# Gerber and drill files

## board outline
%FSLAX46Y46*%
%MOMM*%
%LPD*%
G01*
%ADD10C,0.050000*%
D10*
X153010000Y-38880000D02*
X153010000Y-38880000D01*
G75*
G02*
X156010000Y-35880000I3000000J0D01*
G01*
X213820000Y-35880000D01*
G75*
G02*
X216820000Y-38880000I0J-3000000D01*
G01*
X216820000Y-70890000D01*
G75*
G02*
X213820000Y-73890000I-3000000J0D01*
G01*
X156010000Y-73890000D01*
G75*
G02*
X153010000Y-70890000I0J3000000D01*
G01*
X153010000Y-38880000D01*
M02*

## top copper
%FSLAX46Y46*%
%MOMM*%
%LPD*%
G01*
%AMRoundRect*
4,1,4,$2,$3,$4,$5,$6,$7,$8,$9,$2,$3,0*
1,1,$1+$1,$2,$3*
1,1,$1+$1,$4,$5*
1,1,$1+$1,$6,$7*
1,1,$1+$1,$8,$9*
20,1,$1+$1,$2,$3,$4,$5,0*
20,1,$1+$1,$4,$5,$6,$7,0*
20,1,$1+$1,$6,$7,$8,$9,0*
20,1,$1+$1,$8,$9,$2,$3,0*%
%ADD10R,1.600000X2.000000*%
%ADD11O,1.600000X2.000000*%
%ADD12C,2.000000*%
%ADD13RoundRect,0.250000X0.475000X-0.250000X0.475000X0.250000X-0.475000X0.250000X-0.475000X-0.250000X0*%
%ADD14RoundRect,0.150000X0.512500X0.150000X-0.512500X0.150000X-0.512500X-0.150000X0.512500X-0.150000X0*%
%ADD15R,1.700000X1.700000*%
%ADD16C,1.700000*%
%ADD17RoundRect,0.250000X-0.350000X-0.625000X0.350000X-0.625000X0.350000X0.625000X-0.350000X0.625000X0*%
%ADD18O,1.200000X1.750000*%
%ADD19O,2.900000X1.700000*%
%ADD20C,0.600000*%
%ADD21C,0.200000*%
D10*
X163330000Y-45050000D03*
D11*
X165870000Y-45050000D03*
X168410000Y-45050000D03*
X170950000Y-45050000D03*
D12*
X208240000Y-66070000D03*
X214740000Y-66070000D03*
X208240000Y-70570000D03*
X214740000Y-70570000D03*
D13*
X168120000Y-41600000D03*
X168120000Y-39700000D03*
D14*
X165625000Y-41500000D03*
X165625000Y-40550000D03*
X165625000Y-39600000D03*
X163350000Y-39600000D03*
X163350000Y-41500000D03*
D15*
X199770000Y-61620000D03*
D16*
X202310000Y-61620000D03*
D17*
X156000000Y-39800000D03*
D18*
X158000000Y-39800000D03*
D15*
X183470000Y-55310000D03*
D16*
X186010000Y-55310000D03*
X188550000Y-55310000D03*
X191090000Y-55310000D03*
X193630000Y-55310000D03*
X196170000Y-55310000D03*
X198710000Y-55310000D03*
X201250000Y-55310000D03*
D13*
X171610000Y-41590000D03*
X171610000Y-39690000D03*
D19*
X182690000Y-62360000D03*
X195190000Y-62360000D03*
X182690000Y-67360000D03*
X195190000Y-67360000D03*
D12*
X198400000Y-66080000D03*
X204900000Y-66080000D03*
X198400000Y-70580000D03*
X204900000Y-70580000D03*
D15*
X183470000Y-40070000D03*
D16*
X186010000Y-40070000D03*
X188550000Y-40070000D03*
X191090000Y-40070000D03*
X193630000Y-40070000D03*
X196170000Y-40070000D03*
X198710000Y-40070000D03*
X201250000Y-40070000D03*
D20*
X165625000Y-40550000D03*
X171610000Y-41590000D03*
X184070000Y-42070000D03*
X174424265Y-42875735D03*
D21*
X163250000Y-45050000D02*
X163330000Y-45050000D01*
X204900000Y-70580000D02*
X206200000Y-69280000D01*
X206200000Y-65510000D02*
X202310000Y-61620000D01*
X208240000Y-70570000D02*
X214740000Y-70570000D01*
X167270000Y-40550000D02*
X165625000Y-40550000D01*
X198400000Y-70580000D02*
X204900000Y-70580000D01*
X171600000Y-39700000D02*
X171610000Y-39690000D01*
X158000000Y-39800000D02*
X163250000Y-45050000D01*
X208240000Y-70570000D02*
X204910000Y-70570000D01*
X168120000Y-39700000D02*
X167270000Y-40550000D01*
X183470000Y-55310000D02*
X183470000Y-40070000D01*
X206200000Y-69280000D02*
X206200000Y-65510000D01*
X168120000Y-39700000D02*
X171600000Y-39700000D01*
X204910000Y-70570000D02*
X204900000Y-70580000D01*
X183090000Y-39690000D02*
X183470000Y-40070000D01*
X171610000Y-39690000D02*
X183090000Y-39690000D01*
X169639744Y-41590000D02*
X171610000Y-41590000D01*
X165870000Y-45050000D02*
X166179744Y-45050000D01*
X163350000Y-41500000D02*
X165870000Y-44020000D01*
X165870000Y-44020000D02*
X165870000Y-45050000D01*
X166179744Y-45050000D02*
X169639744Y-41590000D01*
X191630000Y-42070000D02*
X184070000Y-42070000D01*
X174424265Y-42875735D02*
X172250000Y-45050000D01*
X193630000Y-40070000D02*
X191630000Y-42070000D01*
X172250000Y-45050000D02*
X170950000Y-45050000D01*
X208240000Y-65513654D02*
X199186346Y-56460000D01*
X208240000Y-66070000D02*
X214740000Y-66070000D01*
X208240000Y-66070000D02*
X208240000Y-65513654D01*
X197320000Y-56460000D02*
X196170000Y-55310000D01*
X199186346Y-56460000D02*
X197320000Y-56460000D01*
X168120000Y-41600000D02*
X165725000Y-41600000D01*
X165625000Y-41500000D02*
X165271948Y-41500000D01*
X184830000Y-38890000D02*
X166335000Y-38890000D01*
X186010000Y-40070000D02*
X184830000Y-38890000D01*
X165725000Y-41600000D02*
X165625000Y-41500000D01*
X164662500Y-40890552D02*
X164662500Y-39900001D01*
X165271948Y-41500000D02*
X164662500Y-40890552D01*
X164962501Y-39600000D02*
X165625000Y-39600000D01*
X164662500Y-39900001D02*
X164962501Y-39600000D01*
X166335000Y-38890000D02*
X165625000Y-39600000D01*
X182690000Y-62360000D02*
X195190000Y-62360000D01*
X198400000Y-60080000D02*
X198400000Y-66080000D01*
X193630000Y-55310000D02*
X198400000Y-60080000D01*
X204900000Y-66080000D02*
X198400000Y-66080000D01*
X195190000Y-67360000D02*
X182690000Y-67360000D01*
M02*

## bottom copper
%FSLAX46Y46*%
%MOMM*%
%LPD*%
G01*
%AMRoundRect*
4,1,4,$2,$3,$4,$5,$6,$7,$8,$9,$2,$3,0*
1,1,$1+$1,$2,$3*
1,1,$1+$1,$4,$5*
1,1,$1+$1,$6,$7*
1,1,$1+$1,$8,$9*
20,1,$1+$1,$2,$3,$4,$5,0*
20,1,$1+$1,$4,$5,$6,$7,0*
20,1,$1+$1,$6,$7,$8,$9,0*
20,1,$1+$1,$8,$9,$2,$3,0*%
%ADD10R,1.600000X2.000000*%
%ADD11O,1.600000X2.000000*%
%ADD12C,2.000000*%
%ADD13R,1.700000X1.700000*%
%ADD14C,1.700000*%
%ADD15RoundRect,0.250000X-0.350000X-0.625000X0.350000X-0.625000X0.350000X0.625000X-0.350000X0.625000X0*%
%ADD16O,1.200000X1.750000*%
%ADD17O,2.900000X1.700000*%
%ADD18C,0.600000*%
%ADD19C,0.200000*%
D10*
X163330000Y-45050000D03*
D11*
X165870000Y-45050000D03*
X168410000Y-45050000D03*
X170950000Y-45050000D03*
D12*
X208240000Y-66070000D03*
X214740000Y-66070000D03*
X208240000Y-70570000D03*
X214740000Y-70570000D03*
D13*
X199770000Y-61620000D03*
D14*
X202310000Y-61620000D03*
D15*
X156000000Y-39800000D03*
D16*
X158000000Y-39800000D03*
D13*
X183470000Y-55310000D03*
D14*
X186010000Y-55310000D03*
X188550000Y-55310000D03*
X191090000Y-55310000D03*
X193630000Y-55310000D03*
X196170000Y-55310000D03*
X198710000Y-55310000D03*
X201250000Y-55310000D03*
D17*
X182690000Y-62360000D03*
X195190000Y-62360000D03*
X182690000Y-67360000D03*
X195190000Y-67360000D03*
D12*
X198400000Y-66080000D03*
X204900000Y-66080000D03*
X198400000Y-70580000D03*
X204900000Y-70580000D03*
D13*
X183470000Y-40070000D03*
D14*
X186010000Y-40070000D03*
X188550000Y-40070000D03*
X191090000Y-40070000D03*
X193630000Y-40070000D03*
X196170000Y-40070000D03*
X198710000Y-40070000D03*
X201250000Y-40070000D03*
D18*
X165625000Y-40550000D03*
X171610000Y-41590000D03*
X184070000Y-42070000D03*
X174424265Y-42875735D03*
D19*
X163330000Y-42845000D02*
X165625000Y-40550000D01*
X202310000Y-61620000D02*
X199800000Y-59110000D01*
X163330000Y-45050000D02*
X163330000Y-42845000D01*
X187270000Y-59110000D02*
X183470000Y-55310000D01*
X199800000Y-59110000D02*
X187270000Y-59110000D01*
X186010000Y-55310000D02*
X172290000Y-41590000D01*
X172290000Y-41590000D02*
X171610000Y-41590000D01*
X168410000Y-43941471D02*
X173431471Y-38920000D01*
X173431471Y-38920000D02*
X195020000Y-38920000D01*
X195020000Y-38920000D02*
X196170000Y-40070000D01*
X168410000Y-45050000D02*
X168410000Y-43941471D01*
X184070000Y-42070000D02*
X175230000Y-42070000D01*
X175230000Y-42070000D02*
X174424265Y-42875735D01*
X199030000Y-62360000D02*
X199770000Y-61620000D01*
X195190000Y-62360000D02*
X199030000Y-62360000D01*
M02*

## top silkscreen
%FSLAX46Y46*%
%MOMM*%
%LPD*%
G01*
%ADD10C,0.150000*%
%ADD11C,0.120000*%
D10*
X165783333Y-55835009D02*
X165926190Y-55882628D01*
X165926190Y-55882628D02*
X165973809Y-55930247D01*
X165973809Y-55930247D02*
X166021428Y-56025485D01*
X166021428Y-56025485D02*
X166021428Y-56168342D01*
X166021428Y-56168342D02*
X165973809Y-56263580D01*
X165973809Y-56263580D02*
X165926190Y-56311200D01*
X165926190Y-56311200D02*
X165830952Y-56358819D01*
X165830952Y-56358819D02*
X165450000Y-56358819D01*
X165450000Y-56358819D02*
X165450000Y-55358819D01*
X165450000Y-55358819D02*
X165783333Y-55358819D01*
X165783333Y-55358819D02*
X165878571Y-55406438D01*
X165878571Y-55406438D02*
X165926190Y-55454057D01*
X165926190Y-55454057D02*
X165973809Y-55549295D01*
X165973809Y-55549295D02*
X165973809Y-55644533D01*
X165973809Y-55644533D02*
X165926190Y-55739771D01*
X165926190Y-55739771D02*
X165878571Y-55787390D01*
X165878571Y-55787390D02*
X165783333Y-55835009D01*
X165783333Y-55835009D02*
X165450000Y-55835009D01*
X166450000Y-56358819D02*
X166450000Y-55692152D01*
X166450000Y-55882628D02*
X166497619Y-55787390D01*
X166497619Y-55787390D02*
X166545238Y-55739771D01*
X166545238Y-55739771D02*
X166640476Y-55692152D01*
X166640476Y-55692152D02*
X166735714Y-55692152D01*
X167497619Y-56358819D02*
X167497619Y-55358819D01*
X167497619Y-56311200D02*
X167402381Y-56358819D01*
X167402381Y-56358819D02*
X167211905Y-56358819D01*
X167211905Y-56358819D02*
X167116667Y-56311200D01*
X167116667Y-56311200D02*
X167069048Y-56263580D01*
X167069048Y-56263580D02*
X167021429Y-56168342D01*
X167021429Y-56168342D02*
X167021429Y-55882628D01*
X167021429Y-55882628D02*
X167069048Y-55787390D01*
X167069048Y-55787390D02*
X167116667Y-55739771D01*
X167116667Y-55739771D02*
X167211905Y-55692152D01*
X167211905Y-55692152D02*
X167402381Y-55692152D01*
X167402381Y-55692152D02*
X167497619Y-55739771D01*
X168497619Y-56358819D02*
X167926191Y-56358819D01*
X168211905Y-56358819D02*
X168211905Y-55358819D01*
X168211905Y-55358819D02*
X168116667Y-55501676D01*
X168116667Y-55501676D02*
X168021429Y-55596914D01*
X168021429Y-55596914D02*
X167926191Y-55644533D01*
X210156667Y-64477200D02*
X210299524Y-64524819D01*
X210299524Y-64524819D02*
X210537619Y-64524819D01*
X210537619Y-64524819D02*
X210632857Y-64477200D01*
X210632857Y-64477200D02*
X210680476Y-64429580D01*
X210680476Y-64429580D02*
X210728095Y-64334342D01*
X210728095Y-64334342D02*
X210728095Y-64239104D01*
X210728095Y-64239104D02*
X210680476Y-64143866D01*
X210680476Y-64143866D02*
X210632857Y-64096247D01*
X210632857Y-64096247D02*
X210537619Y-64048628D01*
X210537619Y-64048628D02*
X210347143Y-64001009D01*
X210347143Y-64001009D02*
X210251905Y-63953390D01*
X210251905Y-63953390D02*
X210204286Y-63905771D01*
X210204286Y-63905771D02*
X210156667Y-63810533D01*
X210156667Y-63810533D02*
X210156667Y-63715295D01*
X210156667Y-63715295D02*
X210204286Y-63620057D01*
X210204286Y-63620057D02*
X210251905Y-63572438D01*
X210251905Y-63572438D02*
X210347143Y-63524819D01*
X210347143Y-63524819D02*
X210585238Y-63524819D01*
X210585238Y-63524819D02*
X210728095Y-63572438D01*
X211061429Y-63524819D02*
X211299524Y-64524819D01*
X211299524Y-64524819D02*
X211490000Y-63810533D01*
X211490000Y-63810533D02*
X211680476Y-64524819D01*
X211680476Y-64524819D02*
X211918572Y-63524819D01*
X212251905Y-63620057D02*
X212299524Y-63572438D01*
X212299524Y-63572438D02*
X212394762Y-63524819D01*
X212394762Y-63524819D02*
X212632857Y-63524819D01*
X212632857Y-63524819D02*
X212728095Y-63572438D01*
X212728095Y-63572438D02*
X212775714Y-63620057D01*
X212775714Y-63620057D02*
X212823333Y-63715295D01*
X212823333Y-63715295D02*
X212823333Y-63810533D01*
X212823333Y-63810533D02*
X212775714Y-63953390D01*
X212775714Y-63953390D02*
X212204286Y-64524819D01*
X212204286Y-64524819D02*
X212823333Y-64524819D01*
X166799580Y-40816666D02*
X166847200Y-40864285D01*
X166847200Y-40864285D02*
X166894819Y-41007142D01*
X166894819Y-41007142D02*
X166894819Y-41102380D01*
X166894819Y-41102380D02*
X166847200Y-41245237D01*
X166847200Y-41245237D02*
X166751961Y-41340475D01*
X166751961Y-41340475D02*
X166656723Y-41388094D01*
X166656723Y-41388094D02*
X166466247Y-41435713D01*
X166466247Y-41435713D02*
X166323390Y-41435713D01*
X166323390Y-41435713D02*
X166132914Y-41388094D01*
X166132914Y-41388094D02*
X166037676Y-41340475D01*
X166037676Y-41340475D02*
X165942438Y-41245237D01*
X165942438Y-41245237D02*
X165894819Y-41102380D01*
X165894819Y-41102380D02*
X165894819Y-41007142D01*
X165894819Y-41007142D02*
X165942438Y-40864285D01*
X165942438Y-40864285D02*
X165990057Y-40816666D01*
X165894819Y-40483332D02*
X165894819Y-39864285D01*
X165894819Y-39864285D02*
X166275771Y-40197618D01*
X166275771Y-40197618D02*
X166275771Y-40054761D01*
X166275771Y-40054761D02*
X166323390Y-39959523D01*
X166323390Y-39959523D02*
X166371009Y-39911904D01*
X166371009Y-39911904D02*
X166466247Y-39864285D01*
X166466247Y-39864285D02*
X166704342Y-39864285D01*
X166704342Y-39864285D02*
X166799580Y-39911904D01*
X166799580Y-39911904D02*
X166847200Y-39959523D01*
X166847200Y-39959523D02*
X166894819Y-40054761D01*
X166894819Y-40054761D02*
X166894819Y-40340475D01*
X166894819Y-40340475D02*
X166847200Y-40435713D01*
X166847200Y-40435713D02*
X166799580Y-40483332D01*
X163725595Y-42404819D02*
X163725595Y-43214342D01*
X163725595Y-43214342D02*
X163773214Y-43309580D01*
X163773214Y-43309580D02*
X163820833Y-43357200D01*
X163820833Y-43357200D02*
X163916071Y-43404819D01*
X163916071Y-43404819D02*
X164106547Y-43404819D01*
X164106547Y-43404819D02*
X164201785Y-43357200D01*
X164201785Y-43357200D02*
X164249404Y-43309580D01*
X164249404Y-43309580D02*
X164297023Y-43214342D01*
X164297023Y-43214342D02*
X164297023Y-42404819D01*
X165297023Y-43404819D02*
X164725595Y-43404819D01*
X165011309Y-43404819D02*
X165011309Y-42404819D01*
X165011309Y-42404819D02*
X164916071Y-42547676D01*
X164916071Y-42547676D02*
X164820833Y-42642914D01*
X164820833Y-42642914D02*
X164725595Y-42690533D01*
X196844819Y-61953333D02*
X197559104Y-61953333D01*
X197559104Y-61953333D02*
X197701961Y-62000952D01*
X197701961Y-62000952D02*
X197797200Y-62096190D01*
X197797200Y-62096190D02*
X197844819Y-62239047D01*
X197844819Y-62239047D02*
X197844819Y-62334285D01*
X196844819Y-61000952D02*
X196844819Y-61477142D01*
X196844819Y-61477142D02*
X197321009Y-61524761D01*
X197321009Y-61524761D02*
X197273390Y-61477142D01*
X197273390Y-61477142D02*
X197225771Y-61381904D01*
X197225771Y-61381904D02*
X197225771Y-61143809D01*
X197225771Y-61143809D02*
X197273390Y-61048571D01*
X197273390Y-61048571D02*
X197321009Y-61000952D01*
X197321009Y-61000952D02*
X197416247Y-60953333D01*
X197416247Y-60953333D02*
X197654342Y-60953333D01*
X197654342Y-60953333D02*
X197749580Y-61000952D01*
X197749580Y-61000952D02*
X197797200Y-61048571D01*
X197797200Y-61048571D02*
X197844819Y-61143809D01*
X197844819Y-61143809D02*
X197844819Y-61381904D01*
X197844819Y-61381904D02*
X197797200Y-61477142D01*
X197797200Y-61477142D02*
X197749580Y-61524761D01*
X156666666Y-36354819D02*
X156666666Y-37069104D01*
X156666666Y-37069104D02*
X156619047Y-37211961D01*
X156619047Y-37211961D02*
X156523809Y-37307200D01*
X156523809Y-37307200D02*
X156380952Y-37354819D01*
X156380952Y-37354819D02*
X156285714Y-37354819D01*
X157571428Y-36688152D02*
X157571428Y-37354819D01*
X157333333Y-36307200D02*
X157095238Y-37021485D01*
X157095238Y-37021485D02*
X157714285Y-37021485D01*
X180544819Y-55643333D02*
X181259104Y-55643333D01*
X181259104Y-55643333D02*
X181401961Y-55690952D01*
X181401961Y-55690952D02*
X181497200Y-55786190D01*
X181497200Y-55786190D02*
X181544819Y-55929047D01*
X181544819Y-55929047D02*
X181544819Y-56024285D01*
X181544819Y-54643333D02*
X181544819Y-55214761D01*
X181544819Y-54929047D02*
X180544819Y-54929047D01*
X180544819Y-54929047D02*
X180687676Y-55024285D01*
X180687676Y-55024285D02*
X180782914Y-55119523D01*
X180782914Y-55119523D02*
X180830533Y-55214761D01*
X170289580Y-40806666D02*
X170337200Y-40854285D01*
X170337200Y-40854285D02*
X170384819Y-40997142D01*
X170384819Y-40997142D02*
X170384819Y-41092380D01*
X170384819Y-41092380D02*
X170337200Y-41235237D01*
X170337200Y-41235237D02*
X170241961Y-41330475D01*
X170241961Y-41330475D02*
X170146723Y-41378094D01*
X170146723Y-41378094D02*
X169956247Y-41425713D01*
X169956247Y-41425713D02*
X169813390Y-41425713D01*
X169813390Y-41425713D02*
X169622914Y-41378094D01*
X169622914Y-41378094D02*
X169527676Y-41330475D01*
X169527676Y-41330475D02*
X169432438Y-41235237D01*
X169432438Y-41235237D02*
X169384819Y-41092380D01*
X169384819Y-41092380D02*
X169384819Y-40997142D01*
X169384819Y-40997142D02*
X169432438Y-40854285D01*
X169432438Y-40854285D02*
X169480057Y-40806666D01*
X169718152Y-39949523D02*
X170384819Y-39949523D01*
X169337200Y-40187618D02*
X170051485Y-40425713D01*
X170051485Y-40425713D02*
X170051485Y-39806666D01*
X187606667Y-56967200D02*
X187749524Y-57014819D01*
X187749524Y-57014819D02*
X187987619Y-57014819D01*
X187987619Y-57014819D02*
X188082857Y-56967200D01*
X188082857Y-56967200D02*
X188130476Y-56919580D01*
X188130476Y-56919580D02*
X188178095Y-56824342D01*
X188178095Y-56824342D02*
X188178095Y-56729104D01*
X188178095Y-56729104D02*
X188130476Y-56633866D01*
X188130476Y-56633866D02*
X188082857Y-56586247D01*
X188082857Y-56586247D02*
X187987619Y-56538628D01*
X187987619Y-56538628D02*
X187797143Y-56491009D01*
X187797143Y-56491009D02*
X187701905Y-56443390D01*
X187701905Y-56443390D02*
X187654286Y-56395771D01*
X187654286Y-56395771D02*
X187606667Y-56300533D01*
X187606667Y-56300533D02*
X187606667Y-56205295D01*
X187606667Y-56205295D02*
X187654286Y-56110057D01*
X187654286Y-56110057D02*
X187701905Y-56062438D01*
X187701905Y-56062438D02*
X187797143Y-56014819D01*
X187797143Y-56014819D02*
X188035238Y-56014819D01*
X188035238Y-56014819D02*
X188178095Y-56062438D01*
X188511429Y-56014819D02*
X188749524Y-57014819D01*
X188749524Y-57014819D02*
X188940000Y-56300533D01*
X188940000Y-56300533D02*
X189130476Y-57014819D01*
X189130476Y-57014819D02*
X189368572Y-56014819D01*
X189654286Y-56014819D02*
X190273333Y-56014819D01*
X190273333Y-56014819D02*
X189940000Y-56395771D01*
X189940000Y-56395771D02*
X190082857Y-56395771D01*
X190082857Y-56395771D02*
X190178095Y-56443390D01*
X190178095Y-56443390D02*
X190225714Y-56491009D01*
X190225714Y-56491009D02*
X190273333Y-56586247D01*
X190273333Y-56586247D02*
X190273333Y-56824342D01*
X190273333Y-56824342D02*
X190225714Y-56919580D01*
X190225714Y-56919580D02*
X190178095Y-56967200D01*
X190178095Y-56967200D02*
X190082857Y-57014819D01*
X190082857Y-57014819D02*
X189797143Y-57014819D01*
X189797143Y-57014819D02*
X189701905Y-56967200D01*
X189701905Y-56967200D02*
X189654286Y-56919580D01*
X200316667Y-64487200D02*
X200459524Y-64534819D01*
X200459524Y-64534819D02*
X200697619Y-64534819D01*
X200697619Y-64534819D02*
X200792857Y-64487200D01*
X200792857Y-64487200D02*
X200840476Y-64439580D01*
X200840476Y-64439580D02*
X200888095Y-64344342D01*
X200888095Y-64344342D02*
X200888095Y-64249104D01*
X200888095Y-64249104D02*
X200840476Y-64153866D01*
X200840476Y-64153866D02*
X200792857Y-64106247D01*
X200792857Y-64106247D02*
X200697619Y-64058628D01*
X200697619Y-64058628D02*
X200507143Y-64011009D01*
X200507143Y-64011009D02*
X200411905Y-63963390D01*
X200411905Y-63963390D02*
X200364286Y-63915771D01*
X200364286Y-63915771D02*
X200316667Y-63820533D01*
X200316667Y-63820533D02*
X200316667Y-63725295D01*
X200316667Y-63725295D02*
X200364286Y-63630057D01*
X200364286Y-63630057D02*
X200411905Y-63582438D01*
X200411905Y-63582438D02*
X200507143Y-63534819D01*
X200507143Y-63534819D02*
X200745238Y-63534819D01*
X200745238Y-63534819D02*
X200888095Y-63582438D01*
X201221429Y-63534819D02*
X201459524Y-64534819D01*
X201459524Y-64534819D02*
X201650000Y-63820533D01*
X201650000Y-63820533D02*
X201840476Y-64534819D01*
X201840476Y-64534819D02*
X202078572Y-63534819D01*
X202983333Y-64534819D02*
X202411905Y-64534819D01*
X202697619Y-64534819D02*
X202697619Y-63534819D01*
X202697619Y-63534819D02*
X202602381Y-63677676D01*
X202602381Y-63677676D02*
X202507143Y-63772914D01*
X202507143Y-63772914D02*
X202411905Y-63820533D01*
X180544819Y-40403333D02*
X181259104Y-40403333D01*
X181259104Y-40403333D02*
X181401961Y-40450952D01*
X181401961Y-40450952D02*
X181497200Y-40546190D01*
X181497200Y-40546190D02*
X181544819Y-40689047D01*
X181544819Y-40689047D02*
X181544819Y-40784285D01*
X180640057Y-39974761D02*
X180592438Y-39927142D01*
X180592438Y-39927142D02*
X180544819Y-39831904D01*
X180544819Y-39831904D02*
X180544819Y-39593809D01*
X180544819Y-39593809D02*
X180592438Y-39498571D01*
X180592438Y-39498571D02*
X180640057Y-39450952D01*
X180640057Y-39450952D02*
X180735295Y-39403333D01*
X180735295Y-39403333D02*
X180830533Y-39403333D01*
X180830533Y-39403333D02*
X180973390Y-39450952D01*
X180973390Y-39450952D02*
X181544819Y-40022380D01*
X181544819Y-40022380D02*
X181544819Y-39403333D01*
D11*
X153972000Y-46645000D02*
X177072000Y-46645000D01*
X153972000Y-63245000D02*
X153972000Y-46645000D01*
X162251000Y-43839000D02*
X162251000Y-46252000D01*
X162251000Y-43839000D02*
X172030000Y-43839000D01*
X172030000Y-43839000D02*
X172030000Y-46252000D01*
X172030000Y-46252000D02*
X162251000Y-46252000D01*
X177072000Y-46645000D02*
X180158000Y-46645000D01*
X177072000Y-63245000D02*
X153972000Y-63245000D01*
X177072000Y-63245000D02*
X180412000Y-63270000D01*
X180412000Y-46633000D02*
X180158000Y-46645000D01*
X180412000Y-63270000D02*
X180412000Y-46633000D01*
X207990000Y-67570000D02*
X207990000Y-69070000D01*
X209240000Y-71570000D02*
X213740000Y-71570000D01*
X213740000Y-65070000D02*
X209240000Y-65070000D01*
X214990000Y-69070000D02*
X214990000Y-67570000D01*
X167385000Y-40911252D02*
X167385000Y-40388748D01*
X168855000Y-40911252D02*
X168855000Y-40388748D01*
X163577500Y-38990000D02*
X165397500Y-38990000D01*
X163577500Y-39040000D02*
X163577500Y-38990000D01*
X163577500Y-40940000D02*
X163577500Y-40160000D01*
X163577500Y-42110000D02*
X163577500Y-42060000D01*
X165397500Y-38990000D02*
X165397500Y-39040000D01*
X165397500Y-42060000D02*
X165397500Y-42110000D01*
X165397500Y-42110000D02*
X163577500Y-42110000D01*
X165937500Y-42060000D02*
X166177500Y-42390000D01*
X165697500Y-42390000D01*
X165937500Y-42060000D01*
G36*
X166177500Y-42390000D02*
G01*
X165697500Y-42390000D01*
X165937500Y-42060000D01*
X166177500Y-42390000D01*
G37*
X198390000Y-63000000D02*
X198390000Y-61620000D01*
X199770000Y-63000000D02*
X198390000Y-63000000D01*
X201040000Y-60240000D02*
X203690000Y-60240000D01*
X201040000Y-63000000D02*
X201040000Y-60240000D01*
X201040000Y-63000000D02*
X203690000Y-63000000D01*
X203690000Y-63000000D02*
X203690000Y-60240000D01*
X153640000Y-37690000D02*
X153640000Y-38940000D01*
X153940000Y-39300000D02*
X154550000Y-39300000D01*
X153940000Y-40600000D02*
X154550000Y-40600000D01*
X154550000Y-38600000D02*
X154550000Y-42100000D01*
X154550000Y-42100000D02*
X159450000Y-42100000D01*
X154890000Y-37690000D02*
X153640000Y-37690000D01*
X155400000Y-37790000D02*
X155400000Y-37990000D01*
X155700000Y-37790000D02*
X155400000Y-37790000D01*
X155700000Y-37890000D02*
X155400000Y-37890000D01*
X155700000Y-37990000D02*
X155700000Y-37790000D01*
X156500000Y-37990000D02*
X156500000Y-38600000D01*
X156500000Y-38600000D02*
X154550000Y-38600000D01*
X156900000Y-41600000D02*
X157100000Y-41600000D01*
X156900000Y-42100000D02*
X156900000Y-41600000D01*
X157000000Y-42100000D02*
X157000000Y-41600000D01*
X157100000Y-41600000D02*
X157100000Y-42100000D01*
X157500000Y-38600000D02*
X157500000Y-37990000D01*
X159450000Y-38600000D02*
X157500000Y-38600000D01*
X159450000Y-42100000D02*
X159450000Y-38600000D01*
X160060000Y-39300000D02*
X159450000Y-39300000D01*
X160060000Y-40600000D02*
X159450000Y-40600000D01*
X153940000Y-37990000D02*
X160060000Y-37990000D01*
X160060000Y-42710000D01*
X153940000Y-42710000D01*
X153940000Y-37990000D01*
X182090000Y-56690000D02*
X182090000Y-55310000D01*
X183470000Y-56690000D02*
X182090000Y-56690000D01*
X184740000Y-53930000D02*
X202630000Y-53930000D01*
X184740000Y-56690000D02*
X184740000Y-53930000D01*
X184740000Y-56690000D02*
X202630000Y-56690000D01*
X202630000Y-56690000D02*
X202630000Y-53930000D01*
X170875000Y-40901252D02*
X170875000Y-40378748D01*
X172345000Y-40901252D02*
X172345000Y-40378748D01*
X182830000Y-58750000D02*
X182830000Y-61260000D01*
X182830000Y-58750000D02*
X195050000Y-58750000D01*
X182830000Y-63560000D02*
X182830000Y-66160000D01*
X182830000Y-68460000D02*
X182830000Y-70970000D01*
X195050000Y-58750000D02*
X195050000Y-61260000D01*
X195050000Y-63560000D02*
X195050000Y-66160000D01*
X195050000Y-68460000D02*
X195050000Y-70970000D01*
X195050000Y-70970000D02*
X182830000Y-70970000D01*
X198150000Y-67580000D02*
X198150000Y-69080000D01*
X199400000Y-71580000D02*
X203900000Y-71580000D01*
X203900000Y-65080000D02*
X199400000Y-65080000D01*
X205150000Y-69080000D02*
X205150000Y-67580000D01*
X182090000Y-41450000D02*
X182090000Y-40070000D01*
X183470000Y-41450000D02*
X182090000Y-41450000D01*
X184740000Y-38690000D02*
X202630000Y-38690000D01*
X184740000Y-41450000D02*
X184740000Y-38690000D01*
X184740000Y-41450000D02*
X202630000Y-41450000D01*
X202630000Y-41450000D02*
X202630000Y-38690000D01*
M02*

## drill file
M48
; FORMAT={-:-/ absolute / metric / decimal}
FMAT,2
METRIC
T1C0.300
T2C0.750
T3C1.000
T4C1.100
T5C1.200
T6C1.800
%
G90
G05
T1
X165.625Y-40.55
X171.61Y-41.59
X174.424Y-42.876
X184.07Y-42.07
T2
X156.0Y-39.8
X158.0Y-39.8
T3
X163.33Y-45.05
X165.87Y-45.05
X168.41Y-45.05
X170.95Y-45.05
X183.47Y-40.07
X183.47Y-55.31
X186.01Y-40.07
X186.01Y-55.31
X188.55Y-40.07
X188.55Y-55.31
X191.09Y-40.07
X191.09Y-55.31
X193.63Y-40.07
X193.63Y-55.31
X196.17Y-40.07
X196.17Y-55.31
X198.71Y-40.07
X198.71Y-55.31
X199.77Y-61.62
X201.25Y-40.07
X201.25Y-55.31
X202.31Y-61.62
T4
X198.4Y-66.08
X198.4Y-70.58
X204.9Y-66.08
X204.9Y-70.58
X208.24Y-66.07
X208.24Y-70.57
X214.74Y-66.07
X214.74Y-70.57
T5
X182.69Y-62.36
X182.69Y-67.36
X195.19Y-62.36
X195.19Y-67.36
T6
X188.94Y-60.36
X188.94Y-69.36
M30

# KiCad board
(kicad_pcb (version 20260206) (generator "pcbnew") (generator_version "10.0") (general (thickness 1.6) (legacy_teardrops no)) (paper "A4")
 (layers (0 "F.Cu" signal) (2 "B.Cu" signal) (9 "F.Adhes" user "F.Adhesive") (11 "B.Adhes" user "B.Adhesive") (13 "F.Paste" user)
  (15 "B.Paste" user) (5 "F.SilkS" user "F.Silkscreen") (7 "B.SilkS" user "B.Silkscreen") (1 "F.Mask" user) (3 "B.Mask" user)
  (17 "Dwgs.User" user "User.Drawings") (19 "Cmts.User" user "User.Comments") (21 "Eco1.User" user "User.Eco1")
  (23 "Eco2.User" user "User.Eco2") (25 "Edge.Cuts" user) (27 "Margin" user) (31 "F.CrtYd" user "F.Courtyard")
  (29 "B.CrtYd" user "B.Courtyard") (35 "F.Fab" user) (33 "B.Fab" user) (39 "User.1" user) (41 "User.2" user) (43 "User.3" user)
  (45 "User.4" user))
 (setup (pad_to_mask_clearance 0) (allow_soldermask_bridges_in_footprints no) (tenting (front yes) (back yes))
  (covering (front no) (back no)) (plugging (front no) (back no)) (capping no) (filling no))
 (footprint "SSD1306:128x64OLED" (layer "F.Cu") (at 166.95 55.65)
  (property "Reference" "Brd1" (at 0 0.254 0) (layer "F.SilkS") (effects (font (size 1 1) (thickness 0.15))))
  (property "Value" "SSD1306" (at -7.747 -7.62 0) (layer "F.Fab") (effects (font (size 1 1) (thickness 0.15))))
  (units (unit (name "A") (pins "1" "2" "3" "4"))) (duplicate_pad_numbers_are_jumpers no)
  (fp_line (start -12.978 -9.005) (end 10.122 -9.005) (stroke (width 0.12) (type solid)) (layer "F.SilkS"))
  (fp_line (start -12.978 7.595) (end -12.978 -9.005) (stroke (width 0.12) (type solid)) (layer "F.SilkS"))
  (fp_line (start -4.699 -11.811) (end -4.699 -9.398) (stroke (width 0.12) (type solid)) (layer "F.SilkS"))
  (fp_line (start -4.699 -11.811) (end 5.08 -11.811) (stroke (width 0.12) (type solid)) (layer "F.SilkS"))
  (fp_line (start 5.08 -11.811) (end 5.08 -9.398) (stroke (width 0.12) (type solid)) (layer "F.SilkS"))
  (fp_line (start 5.08 -9.398) (end -4.699 -9.398) (stroke (width 0.12) (type solid)) (layer "F.SilkS"))
  (fp_line (start 10.122 -9.005) (end 13.208 -9.005) (stroke (width 0.12) (type solid)) (layer "F.SilkS"))
  (fp_line (start 10.122 7.595) (end -12.978 7.595) (stroke (width 0.12) (type solid)) (layer "F.SilkS"))
  (fp_line (start 10.122 7.595) (end 13.462 7.62) (stroke (width 0.12) (type solid)) (layer "F.SilkS"))
  (fp_line (start 13.462 -9.017) (end 13.208 -9.005) (stroke (width 0.12) (type solid)) (layer "F.SilkS"))
  (fp_line (start 13.462 7.62) (end 13.462 -9.017) (stroke (width 0.12) (type solid)) (layer "F.SilkS"))
  (pad "1" thru_hole rect (at -3.62 -10.6 90) (size 2 1.6) (drill 1) (layers "*.Cu" "*.Mask") (remove_unused_layers no) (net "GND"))
  (pad "2" thru_hole oval (at -1.08 -10.6 90) (size 2 1.6) (drill 1) (layers "*.Cu" "*.Mask") (remove_unused_layers no) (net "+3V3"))
  (pad "3" thru_hole oval (at 1.46 -10.6 90) (size 2 1.6) (drill 1) (layers "*.Cu" "*.Mask") (remove_unused_layers no) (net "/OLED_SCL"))
  (pad "4" thru_hole oval (at 4 -10.6 90) (size 2 1.6) (drill 1) (layers "*.Cu" "*.Mask") (remove_unused_layers no) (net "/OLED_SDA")))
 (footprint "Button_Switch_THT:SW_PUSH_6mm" (layer "F.Cu") (at 208.24 66.07)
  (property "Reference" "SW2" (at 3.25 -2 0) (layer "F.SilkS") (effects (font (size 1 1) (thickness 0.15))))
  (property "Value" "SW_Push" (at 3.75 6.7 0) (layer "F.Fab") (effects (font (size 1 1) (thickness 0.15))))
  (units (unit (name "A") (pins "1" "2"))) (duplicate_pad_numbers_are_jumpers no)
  (fp_line (start -0.25 1.5) (end -0.25 3) (stroke (width 0.12) (type solid)) (layer "F.SilkS"))
  (fp_line (start 1 5.5) (end 5.5 5.5) (stroke (width 0.12) (type solid)) (layer "F.SilkS"))
  (fp_line (start 5.5 -1) (end 1 -1) (stroke (width 0.12) (type solid)) (layer "F.SilkS"))
  (fp_line (start 6.75 3) (end 6.75 1.5) (stroke (width 0.12) (type solid)) (layer "F.SilkS"))
  (pad "1" thru_hole circle (at 0 0 90) (size 2 2) (drill 1.1) (layers "*.Cu" "*.Mask") (remove_unused_layers no) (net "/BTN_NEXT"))
  (pad "1" thru_hole circle (at 6.5 0 90) (size 2 2) (drill 1.1) (layers "*.Cu" "*.Mask") (remove_unused_layers no) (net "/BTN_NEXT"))
  (pad "2" thru_hole circle (at 0 4.5 90) (size 2 2) (drill 1.1) (layers "*.Cu" "*.Mask") (remove_unused_layers no) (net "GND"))
  (pad "2" thru_hole circle (at 6.5 4.5 90) (size 2 2) (drill 1.1) (layers "*.Cu" "*.Mask") (remove_unused_layers no) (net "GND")))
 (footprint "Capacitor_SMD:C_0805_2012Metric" (layer "F.Cu") (at 168.12 40.65 90)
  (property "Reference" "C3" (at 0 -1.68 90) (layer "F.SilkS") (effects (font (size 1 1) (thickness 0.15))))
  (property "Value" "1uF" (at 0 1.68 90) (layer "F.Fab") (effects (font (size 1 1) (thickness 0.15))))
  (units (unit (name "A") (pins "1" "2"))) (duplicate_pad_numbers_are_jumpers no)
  (fp_line (start -0.261252 -0.735) (end 0.261252 -0.735) (stroke (width 0.12) (type solid)) (layer "F.SilkS"))
  (fp_line (start -0.261252 0.735) (end 0.261252 0.735) (stroke (width 0.12) (type solid)) (layer "F.SilkS"))
  (pad "1" smd roundrect (at -0.95 0 90) (size 1 1.45) (layers "F.Cu" "F.Mask" "F.Paste") (roundrect_rratio 0.25) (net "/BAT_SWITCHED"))
  (pad "2" smd roundrect (at 0.95 0 90) (size 1 1.45) (layers "F.Cu" "F.Mask" "F.Paste") (roundrect_rratio 0.25) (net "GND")))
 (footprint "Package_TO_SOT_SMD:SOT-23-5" (layer "F.Cu") (at 164.4875 40.55 180)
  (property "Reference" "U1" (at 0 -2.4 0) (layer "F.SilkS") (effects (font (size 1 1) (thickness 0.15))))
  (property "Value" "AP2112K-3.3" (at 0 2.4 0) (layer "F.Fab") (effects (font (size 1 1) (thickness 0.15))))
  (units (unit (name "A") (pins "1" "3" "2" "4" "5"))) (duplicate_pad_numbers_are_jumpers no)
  (fp_line (start 0.91 1.56) (end -0.91 1.56) (stroke (width 0.12) (type solid)) (layer "F.SilkS"))
  (fp_line (start 0.91 1.51) (end 0.91 1.56) (stroke (width 0.12) (type solid)) (layer "F.SilkS"))
  (fp_line (start 0.91 -0.39) (end 0.91 0.39) (stroke (width 0.12) (type solid)) (layer "F.SilkS"))
  (fp_line (start 0.91 -1.56) (end 0.91 -1.51) (stroke (width 0.12) (type solid)) (layer "F.SilkS"))
  (fp_line (start -0.91 1.56) (end -0.91 1.51) (stroke (width 0.12) (type solid)) (layer "F.SilkS"))
  (fp_line (start -0.91 -1.51) (end -0.91 -1.56) (stroke (width 0.12) (type solid)) (layer "F.SilkS"))
  (fp_line (start -0.91 -1.56) (end 0.91 -1.56) (stroke (width 0.12) (type solid)) (layer "F.SilkS"))
  (fp_poly (pts (xy -1.45 -1.51) (xy -1.69 -1.84) (xy -1.21 -1.84)) (stroke (width 0.12) (type solid)) (fill yes) (layer "F.SilkS"))
  (pad "1" smd roundrect (at -1.1375 -0.95 180) (size 1.325 0.6) (layers "F.Cu" "F.Mask" "F.Paste") (roundrect_rratio 0.25)
   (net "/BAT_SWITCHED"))
  (pad "2" smd roundrect (at -1.1375 0 180) (size 1.325 0.6) (layers "F.Cu" "F.Mask" "F.Paste") (roundrect_rratio 0.25) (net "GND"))
  (pad "3" smd roundrect (at -1.1375 0.95 180) (size 1.325 0.6) (layers "F.Cu" "F.Mask" "F.Paste") (roundrect_rratio 0.25)
   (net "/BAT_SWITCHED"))
  (pad "4" smd roundrect (at 1.1375 0.95 180) (size 1.325 0.6) (layers "F.Cu" "F.Mask" "F.Paste") (roundrect_rratio 0.25)
   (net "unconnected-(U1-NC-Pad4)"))
  (pad "5" smd roundrect (at 1.1375 -0.95 180) (size 1.325 0.6) (layers "F.Cu" "F.Mask" "F.Paste") (roundrect_rratio 0.25) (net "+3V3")))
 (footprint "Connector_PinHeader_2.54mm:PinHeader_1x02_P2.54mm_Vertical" (layer "F.Cu") (at 199.77 61.62 90)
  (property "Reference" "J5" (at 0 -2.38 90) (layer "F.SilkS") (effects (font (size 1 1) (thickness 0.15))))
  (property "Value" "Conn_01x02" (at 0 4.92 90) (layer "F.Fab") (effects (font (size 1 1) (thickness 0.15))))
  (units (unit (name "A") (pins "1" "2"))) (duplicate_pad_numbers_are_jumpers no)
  (fp_line (start -1.38 -1.38) (end 0 -1.38) (stroke (width 0.12) (type solid)) (layer "F.SilkS"))
  (fp_line (start -1.38 0) (end -1.38 -1.38) (stroke (width 0.12) (type solid)) (layer "F.SilkS"))
  (fp_line (start 1.38 1.27) (end 1.38 3.92) (stroke (width 0.12) (type solid)) (layer "F.SilkS"))
  (fp_line (start -1.38 1.27) (end 1.38 1.27) (stroke (width 0.12) (type solid)) (layer "F.SilkS"))
  (fp_line (start -1.38 1.27) (end -1.38 3.92) (stroke (width 0.12) (type solid)) (layer "F.SilkS"))
  (fp_line (start -1.38 3.92) (end 1.38 3.92) (stroke (width 0.12) (type solid)) (layer "F.SilkS"))
  (pad "1" thru_hole rect (at 0 0 90) (size 1.7 1.7) (drill 1) (layers "*.Cu" "*.Mask") (remove_unused_layers no) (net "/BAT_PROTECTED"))
  (pad "2" thru_hole circle (at 0 2.54 90) (size 1.7 1.7) (drill 1) (layers "*.Cu" "*.Mask") (remove_unused_layers no) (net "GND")))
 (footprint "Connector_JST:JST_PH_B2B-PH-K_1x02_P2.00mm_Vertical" (layer "F.Cu") (at 156 39.8)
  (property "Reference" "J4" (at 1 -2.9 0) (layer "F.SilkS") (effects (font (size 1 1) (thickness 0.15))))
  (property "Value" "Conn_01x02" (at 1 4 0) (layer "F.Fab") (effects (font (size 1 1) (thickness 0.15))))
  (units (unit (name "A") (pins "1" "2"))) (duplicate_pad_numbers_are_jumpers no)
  (fp_line (start -2.36 -2.11) (end -2.36 -0.86) (stroke (width 0.12) (type solid)) (layer "F.SilkS"))
  (fp_line (start -2.06 -0.5) (end -1.45 -0.5) (stroke (width 0.12) (type solid)) (layer "F.SilkS"))
  (fp_line (start -2.06 0.8) (end -1.45 0.8) (stroke (width 0.12) (type solid)) (layer "F.SilkS"))
  (fp_line (start -1.45 -1.2) (end -1.45 2.3) (stroke (width 0.12) (type solid)) (layer "F.SilkS"))
  (fp_line (start -1.45 2.3) (end 3.45 2.3) (stroke (width 0.12) (type solid)) (layer "F.SilkS"))
  (fp_line (start -1.11 -2.11) (end -2.36 -2.11) (stroke (width 0.12) (type solid)) (layer "F.SilkS"))
  (fp_line (start -0.6 -2.01) (end -0.6 -1.81) (stroke (width 0.12) (type solid)) (layer "F.SilkS"))
  (fp_line (start -0.3 -2.01) (end -0.6 -2.01) (stroke (width 0.12) (type solid)) (layer "F.SilkS"))
  (fp_line (start -0.3 -1.91) (end -0.6 -1.91) (stroke (width 0.12) (type solid)) (layer "F.SilkS"))
  (fp_line (start -0.3 -1.81) (end -0.3 -2.01) (stroke (width 0.12) (type solid)) (layer "F.SilkS"))
  (fp_line (start 0.5 -1.81) (end 0.5 -1.2) (stroke (width 0.12) (type solid)) (layer "F.SilkS"))
  (fp_line (start 0.5 -1.2) (end -1.45 -1.2) (stroke (width 0.12) (type solid)) (layer "F.SilkS"))
  (fp_line (start 0.9 1.8) (end 1.1 1.8) (stroke (width 0.12) (type solid)) (layer "F.SilkS"))
  (fp_line (start 0.9 2.3) (end 0.9 1.8) (stroke (width 0.12) (type solid)) (layer "F.SilkS"))
  (fp_line (start 1 2.3) (end 1 1.8) (stroke (width 0.12) (type solid)) (layer "F.SilkS"))
  (fp_line (start 1.1 1.8) (end 1.1 2.3) (stroke (width 0.12) (type solid)) (layer "F.SilkS"))
  (fp_line (start 1.5 -1.2) (end 1.5 -1.81) (stroke (width 0.12) (type solid)) (layer "F.SilkS"))
  (fp_line (start 3.45 -1.2) (end 1.5 -1.2) (stroke (width 0.12) (type solid)) (layer "F.SilkS"))
  (fp_line (start 3.45 2.3) (end 3.45 -1.2) (stroke (width 0.12) (type solid)) (layer "F.SilkS"))
  (fp_line (start 4.06 -0.5) (end 3.45 -0.5) (stroke (width 0.12) (type solid)) (layer "F.SilkS"))
  (fp_line (start 4.06 0.8) (end 3.45 0.8) (stroke (width 0.12) (type solid)) (layer "F.SilkS"))
  (fp_rect (start -2.06 -1.81) (end 4.06 2.91) (stroke (width 0.12) (type solid)) (fill no) (layer "F.SilkS"))
  (pad "1" thru_hole roundrect (at 0 0) (size 1.2 1.75) (drill 0.75) (layers "*.Cu" "*.Mask") (remove_unused_layers no)
   (roundrect_rratio 0.208333) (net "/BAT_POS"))
  (pad "2" thru_hole oval (at 2 0) (size 1.2 1.75) (drill 0.75) (layers "*.Cu" "*.Mask") (remove_unused_layers no) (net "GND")))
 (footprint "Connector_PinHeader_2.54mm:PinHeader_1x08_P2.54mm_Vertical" (layer "F.Cu") (at 183.47 55.31 90)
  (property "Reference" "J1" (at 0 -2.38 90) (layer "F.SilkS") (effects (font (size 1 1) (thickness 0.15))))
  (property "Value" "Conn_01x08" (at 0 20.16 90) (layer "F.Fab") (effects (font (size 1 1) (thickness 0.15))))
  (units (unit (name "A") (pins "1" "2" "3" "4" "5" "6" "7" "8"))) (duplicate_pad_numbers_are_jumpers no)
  (fp_line (start -1.38 -1.38) (end 0 -1.38) (stroke (width 0.12) (type solid)) (layer "F.SilkS"))
  (fp_line (start -1.38 0) (end -1.38 -1.38) (stroke (width 0.12) (type solid)) (layer "F.SilkS"))
  (fp_line (start 1.38 1.27) (end 1.38 19.16) (stroke (width 0.12) (type solid)) (layer "F.SilkS"))
  (fp_line (start -1.38 1.27) (end 1.38 1.27) (stroke (width 0.12) (type solid)) (layer "F.SilkS"))
  (fp_line (start -1.38 1.27) (end -1.38 19.16) (stroke (width 0.12) (type solid)) (layer "F.SilkS"))
  (fp_line (start -1.38 19.16) (end 1.38 19.16) (stroke (width 0.12) (type solid)) (layer "F.SilkS"))
  (pad "1" thru_hole rect (at 0 0 90) (size 1.7 1.7) (drill 1) (layers "*.Cu" "*.Mask") (remove_unused_layers no) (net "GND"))
  (pad "2" thru_hole circle (at 0 2.54 90) (size 1.7 1.7) (drill 1) (layers "*.Cu" "*.Mask") (remove_unused_layers no) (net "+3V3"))
  (pad "3" thru_hole circle (at 0 5.08 90) (size 1.7 1.7) (drill 1) (layers "*.Cu" "*.Mask") (remove_unused_layers no) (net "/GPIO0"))
  (pad "4" thru_hole circle (at 0 7.62 90) (size 1.7 1.7) (drill 1) (layers "*.Cu" "*.Mask") (remove_unused_layers no) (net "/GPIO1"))
  (pad "5" thru_hole circle (at 0 10.16 90) (size 1.7 1.7) (drill 1) (layers "*.Cu" "*.Mask") (remove_unused_layers no) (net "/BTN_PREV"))
  (pad "6" thru_hole circle (at 0 12.7 90) (size 1.7 1.7) (drill 1) (layers "*.Cu" "*.Mask") (remove_unused_layers no) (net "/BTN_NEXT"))
  (pad "7" thru_hole circle (at 0 15.24 90) (size 1.7 1.7) (drill 1) (layers "*.Cu" "*.Mask") (remove_unused_layers no) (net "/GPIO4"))
  (pad "8" thru_hole circle (at 0 17.78 90) (size 1.7 1.7) (drill 1) (layers "*.Cu" "*.Mask") (remove_unused_layers no) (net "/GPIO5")))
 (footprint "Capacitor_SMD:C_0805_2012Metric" (layer "F.Cu") (at 171.61 40.64 90)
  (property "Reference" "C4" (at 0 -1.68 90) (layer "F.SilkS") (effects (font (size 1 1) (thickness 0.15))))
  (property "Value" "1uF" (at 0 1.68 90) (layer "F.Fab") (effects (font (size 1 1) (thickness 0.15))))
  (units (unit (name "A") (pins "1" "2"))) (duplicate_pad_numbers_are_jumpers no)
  (fp_line (start -0.261252 -0.735) (end 0.261252 -0.735) (stroke (width 0.12) (type solid)) (layer "F.SilkS"))
  (fp_line (start -0.261252 0.735) (end 0.261252 0.735) (stroke (width 0.12) (type solid)) (layer "F.SilkS"))
  (pad "1" smd roundrect (at -0.95 0 90) (size 1 1.45) (layers "F.Cu" "F.Mask" "F.Paste") (roundrect_rratio 0.25) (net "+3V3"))
  (pad "2" smd roundrect (at 0.95 0 90) (size 1 1.45) (layers "F.Cu" "F.Mask" "F.Paste") (roundrect_rratio 0.25) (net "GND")))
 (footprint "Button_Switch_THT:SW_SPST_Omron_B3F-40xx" (layer "F.Cu") (at 182.69 62.36)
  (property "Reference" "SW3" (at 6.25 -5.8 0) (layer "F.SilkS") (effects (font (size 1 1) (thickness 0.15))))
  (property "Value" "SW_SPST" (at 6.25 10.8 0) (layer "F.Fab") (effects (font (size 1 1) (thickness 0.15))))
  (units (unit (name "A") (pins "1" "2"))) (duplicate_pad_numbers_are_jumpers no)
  (fp_line (start 0.14 -3.61) (end 0.14 -1.1) (stroke (width 0.12) (type default)) (layer "F.SilkS"))
  (fp_line (start 0.14 -3.61) (end 12.36 -3.61) (stroke (width 0.12) (type default)) (layer "F.SilkS"))
  (fp_line (start 0.14 1.2) (end 0.14 3.8) (stroke (width 0.12) (type default)) (layer "F.SilkS"))
  (fp_line (start 0.14 6.1) (end 0.14 8.61) (stroke (width 0.12) (type default)) (layer "F.SilkS"))
  (fp_line (start 12.36 -3.61) (end 12.36 -1.1) (stroke (width 0.12) (type default)) (layer "F.SilkS"))
  (fp_line (start 12.36 1.2) (end 12.36 3.8) (stroke (width 0.12) (type default)) (layer "F.SilkS"))
  (fp_line (start 12.36 6.1) (end 12.36 8.61) (stroke (width 0.12) (type default)) (layer "F.SilkS"))
  (fp_line (start 12.36 8.61) (end 0.14 8.61) (stroke (width 0.12) (type default)) (layer "F.SilkS"))
  (pad "" np_thru_hole circle (at 6.25 -2) (size 1.8 1.8) (drill 1.8) (layers "*.Cu" "*.Mask"))
  (pad "" np_thru_hole circle (at 6.25 7) (size 1.8 1.8) (drill 1.8) (layers "*.Cu" "*.Mask"))
  (pad "1" thru_hole oval (at 0 0) (size 2.9 1.7) (drill 1.2) (layers "*.Cu" "*.Mask") (remove_unused_layers no) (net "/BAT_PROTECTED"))
  (pad "1" thru_hole oval (at 12.5 0) (size 2.9 1.7) (drill 1.2) (layers "*.Cu" "*.Mask") (remove_unused_layers no) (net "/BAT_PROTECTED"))
  (pad "2" thru_hole oval (at 0 5) (size 2.9 1.7) (drill 1.2) (layers "*.Cu" "*.Mask") (remove_unused_layers no) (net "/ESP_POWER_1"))
  (pad "2" thru_hole oval (at 12.5 5) (size 2.9 1.7) (drill 1.2) (layers "*.Cu" "*.Mask") (remove_unused_layers no) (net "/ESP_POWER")))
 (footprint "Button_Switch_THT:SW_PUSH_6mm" (layer "F.Cu") (at 198.4 66.08)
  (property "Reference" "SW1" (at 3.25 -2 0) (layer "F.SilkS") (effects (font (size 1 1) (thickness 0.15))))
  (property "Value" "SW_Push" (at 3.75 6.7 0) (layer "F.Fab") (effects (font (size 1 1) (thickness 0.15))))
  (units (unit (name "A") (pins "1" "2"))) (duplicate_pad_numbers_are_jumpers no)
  (fp_line (start -0.25 1.5) (end -0.25 3) (stroke (width 0.12) (type solid)) (layer "F.SilkS"))
  (fp_line (start 1 5.5) (end 5.5 5.5) (stroke (width 0.12) (type solid)) (layer "F.SilkS"))
  (fp_line (start 5.5 -1) (end 1 -1) (stroke (width 0.12) (type solid)) (layer "F.SilkS"))
  (fp_line (start 6.75 3) (end 6.75 1.5) (stroke (width 0.12) (type solid)) (layer "F.SilkS"))
  (pad "1" thru_hole circle (at 0 0 90) (size 2 2) (drill 1.1) (layers "*.Cu" "*.Mask") (remove_unused_layers no) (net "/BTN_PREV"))
  (pad "1" thru_hole circle (at 6.5 0 90) (size 2 2) (drill 1.1) (layers "*.Cu" "*.Mask") (remove_unused_layers no) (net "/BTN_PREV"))
  (pad "2" thru_hole circle (at 0 4.5 90) (size 2 2) (drill 1.1) (layers "*.Cu" "*.Mask") (remove_unused_layers no) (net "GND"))
  (pad "2" thru_hole circle (at 6.5 4.5 90) (size 2 2) (drill 1.1) (layers "*.Cu" "*.Mask") (remove_unused_layers no) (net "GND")))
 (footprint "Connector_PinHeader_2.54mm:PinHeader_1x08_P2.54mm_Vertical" (layer "F.Cu") (at 183.47 40.07 90)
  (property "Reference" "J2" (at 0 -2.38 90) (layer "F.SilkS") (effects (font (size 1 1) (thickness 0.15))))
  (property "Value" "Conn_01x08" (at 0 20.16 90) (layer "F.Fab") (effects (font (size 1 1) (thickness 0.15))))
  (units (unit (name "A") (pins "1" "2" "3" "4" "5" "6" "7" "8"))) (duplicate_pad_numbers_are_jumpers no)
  (fp_line (start -1.38 -1.38) (end 0 -1.38) (stroke (width 0.12) (type solid)) (layer "F.SilkS"))
  (fp_line (start -1.38 0) (end -1.38 -1.38) (stroke (width 0.12) (type solid)) (layer "F.SilkS"))
  (fp_line (start 1.38 1.27) (end 1.38 19.16) (stroke (width 0.12) (type solid)) (layer "F.SilkS"))
  (fp_line (start -1.38 1.27) (end 1.38 1.27) (stroke (width 0.12) (type solid)) (layer "F.SilkS"))
  (fp_line (start -1.38 1.27) (end -1.38 19.16) (stroke (width 0.12) (type solid)) (layer "F.SilkS"))
  (fp_line (start -1.38 19.16) (end 1.38 19.16) (stroke (width 0.12) (type solid)) (layer "F.SilkS"))
  (pad "1" thru_hole rect (at 0 0 90) (size 1.7 1.7) (drill 1) (layers "*.Cu" "*.Mask") (remove_unused_layers no) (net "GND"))
  (pad "2" thru_hole circle (at 0 2.54 90) (size 1.7 1.7) (drill 1) (layers "*.Cu" "*.Mask") (remove_unused_layers no) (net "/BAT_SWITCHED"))
  (pad "3" thru_hole circle (at 0 5.08 90) (size 1.7 1.7) (drill 1) (layers "*.Cu" "*.Mask") (remove_unused_layers no) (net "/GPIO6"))
  (pad "4" thru_hole circle (at 0 7.62 90) (size 1.7 1.7) (drill 1) (layers "*.Cu" "*.Mask") (remove_unused_layers no) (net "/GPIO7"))
  (pad "5" thru_hole circle (at 0 10.16 90) (size 1.7 1.7) (drill 1) (layers "*.Cu" "*.Mask") (remove_unused_layers no) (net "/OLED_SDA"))
  (pad "6" thru_hole circle (at 0 12.7 90) (size 1.7 1.7) (drill 1) (layers "*.Cu" "*.Mask") (remove_unused_layers no) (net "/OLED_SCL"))
  (pad "7" thru_hole circle (at 0 15.24 90) (size 1.7 1.7) (drill 1) (layers "*.Cu" "*.Mask") (remove_unused_layers no) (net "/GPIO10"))
  (pad "8" thru_hole circle (at 0 17.78 90) (size 1.7 1.7) (drill 1) (layers "*.Cu" "*.Mask") (remove_unused_layers no) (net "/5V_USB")))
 (gr_rect (start 153.01 35.88) (end 216.82 73.89) (radius 3) (stroke (width 0.05) (type solid)) (fill no) (layer "Edge.Cuts"))
 (segment (start 163.25 45.05) (end 163.33 45.05) (width 0.2) (layer "F.Cu") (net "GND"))
 (segment (start 204.9 70.58) (end 206.2 69.28) (width 0.2) (layer "F.Cu") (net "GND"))
 (segment (start 206.2 65.51) (end 202.31 61.62) (width 0.2) (layer "F.Cu") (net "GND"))
 (segment (start 208.24 70.57) (end 214.74 70.57) (width 0.2) (layer "F.Cu") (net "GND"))
 (segment (start 167.27 40.55) (end 165.625 40.55) (width 0.2) (layer "F.Cu") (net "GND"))
 (segment (start 198.4 70.58) (end 204.9 70.58) (width 0.2) (layer "F.Cu") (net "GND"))
 (segment (start 171.6 39.7) (end 171.61 39.69) (width 0.2) (layer "F.Cu") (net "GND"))
 (segment (start 158 39.8) (end 163.25 45.05) (width 0.2) (layer "F.Cu") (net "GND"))
 (segment (start 208.24 70.57) (end 204.91 70.57) (width 0.2) (layer "F.Cu") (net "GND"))
 (segment (start 168.12 39.7) (end 167.27 40.55) (width 0.2) (layer "F.Cu") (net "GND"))
 (segment (start 183.47 55.31) (end 183.47 40.07) (width 0.2) (layer "F.Cu") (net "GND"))
 (segment (start 206.2 69.28) (end 206.2 65.51) (width 0.2) (layer "F.Cu") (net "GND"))
 (segment (start 168.12 39.7) (end 171.6 39.7) (width 0.2) (layer "F.Cu") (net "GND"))
 (segment (start 204.91 70.57) (end 204.9 70.58) (width 0.2) (layer "F.Cu") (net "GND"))
 (segment (start 183.09 39.69) (end 183.47 40.07) (width 0.2) (layer "F.Cu") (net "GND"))
 (segment (start 171.61 39.69) (end 183.09 39.69) (width 0.2) (layer "F.Cu") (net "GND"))
 (via (at 165.625 40.55) (size 0.6) (drill 0.3) (layers "F.Cu" "B.Cu") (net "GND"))
 (segment (start 163.33 42.845) (end 165.625 40.55) (width 0.2) (layer "B.Cu") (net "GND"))
 (segment (start 202.31 61.62) (end 199.8 59.11) (width 0.2) (layer "B.Cu") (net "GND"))
 (segment (start 163.33 45.05) (end 163.33 42.845) (width 0.2) (layer "B.Cu") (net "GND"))
 (segment (start 187.27 59.11) (end 183.47 55.31) (width 0.2) (layer "B.Cu") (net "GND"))
 (segment (start 199.8 59.11) (end 187.27 59.11) (width 0.2) (layer "B.Cu") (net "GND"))
 (segment (start 169.639744 41.59) (end 171.61 41.59) (width 0.2) (layer "F.Cu") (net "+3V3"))
 (segment (start 165.87 45.05) (end 166.179744 45.05) (width 0.2) (layer "F.Cu") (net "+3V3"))
 (segment (start 163.35 41.5) (end 165.87 44.02) (width 0.2) (layer "F.Cu") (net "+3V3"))
 (segment (start 165.87 44.02) (end 165.87 45.05) (width 0.2) (layer "F.Cu") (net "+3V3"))
 (segment (start 166.179744 45.05) (end 169.639744 41.59) (width 0.2) (layer "F.Cu") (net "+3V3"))
 (via (at 171.61 41.59) (size 0.6) (drill 0.3) (layers "F.Cu" "B.Cu") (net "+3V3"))
 (segment (start 186.01 55.31) (end 172.29 41.59) (width 0.2) (layer "B.Cu") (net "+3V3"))
 (segment (start 172.29 41.59) (end 171.61 41.59) (width 0.2) (layer "B.Cu") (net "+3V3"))
 (segment (start 168.41 43.941471) (end 173.431471 38.92) (width 0.2) (layer "B.Cu") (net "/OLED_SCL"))
 (segment (start 173.431471 38.92) (end 195.02 38.92) (width 0.2) (layer "B.Cu") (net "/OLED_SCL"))
 (segment (start 195.02 38.92) (end 196.17 40.07) (width 0.2) (layer "B.Cu") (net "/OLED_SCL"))
 (segment (start 168.41 45.05) (end 168.41 43.941471) (width 0.2) (layer "B.Cu") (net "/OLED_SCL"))
 (segment (start 191.63 42.07) (end 184.07 42.07) (width 0.2) (layer "F.Cu") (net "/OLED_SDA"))
 (segment (start 174.424265 42.875735) (end 172.25 45.05) (width 0.2) (layer "F.Cu") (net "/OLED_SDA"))
 (segment (start 193.63 40.07) (end 191.63 42.07) (width 0.2) (layer "F.Cu") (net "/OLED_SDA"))
 (segment (start 172.25 45.05) (end 170.95 45.05) (width 0.2) (layer "F.Cu") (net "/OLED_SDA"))
 (via (at 184.07 42.07) (size 0.6) (drill 0.3) (layers "F.Cu" "B.Cu") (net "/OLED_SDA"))
 (via (at 174.424265 42.875735) (size 0.6) (drill 0.3) (layers "F.Cu" "B.Cu") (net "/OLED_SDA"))
 (segment (start 184.07 42.07) (end 175.23 42.07) (width 0.2) (layer "B.Cu") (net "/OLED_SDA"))
 (segment (start 175.23 42.07) (end 174.424265 42.875735) (width 0.2) (layer "B.Cu") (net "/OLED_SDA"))
 (segment (start 208.24 65.513654) (end 199.186346 56.46) (width 0.2) (layer "F.Cu") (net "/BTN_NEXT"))
 (segment (start 208.24 66.07) (end 214.74 66.07) (width 0.2) (layer "F.Cu") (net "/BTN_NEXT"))
 (segment (start 208.24 66.07) (end 208.24 65.513654) (width 0.2) (layer "F.Cu") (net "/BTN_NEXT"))
 (segment (start 197.32 56.46) (end 196.17 55.31) (width 0.2) (layer "F.Cu") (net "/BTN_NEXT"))
 (segment (start 199.186346 56.46) (end 197.32 56.46) (width 0.2) (layer "F.Cu") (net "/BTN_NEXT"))
 (segment (start 168.12 41.6) (end 165.725 41.6) (width 0.2) (layer "F.Cu") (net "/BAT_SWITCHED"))
 (segment (start 165.625 41.5) (end 165.271948 41.5) (width 0.2) (layer "F.Cu") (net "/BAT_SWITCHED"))
 (segment (start 184.83 38.89) (end 166.335 38.89) (width 0.2) (layer "F.Cu") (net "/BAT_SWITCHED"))
 (segment (start 186.01 40.07) (end 184.83 38.89) (width 0.2) (layer "F.Cu") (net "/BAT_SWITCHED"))
 (segment (start 165.725 41.6) (end 165.625 41.5) (width 0.2) (layer "F.Cu") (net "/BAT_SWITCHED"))
 (segment (start 164.6625 40.890552) (end 164.6625 39.900001) (width 0.2) (layer "F.Cu") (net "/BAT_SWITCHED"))
 (segment (start 165.271948 41.5) (end 164.6625 40.890552) (width 0.2) (layer "F.Cu") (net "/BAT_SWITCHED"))
 (segment (start 164.962501 39.6) (end 165.625 39.6) (width 0.2) (layer "F.Cu") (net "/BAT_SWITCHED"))
 (segment (start 164.6625 39.900001) (end 164.962501 39.6) (width 0.2) (layer "F.Cu") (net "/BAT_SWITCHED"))
 (segment (start 166.335 38.89) (end 165.625 39.6) (width 0.2) (layer "F.Cu") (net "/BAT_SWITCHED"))
 (segment (start 182.69 62.36) (end 195.19 62.36) (width 0.2) (layer "F.Cu") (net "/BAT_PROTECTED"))
 (segment (start 199.03 62.36) (end 199.77 61.62) (width 0.2) (layer "B.Cu") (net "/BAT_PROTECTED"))
 (segment (start 195.19 62.36) (end 199.03 62.36) (width 0.2) (layer "B.Cu") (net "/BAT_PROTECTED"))
 (segment (start 198.4 60.08) (end 198.4 66.08) (width 0.2) (layer "F.Cu") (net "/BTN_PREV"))
 (segment (start 193.63 55.31) (end 198.4 60.08) (width 0.2) (layer "F.Cu") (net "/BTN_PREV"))
 (segment (start 204.9 66.08) (end 198.4 66.08) (width 0.2) (layer "F.Cu") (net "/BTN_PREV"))
 (segment (start 195.19 67.36) (end 182.69 67.36) (width 0.2) (layer "F.Cu") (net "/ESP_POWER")))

